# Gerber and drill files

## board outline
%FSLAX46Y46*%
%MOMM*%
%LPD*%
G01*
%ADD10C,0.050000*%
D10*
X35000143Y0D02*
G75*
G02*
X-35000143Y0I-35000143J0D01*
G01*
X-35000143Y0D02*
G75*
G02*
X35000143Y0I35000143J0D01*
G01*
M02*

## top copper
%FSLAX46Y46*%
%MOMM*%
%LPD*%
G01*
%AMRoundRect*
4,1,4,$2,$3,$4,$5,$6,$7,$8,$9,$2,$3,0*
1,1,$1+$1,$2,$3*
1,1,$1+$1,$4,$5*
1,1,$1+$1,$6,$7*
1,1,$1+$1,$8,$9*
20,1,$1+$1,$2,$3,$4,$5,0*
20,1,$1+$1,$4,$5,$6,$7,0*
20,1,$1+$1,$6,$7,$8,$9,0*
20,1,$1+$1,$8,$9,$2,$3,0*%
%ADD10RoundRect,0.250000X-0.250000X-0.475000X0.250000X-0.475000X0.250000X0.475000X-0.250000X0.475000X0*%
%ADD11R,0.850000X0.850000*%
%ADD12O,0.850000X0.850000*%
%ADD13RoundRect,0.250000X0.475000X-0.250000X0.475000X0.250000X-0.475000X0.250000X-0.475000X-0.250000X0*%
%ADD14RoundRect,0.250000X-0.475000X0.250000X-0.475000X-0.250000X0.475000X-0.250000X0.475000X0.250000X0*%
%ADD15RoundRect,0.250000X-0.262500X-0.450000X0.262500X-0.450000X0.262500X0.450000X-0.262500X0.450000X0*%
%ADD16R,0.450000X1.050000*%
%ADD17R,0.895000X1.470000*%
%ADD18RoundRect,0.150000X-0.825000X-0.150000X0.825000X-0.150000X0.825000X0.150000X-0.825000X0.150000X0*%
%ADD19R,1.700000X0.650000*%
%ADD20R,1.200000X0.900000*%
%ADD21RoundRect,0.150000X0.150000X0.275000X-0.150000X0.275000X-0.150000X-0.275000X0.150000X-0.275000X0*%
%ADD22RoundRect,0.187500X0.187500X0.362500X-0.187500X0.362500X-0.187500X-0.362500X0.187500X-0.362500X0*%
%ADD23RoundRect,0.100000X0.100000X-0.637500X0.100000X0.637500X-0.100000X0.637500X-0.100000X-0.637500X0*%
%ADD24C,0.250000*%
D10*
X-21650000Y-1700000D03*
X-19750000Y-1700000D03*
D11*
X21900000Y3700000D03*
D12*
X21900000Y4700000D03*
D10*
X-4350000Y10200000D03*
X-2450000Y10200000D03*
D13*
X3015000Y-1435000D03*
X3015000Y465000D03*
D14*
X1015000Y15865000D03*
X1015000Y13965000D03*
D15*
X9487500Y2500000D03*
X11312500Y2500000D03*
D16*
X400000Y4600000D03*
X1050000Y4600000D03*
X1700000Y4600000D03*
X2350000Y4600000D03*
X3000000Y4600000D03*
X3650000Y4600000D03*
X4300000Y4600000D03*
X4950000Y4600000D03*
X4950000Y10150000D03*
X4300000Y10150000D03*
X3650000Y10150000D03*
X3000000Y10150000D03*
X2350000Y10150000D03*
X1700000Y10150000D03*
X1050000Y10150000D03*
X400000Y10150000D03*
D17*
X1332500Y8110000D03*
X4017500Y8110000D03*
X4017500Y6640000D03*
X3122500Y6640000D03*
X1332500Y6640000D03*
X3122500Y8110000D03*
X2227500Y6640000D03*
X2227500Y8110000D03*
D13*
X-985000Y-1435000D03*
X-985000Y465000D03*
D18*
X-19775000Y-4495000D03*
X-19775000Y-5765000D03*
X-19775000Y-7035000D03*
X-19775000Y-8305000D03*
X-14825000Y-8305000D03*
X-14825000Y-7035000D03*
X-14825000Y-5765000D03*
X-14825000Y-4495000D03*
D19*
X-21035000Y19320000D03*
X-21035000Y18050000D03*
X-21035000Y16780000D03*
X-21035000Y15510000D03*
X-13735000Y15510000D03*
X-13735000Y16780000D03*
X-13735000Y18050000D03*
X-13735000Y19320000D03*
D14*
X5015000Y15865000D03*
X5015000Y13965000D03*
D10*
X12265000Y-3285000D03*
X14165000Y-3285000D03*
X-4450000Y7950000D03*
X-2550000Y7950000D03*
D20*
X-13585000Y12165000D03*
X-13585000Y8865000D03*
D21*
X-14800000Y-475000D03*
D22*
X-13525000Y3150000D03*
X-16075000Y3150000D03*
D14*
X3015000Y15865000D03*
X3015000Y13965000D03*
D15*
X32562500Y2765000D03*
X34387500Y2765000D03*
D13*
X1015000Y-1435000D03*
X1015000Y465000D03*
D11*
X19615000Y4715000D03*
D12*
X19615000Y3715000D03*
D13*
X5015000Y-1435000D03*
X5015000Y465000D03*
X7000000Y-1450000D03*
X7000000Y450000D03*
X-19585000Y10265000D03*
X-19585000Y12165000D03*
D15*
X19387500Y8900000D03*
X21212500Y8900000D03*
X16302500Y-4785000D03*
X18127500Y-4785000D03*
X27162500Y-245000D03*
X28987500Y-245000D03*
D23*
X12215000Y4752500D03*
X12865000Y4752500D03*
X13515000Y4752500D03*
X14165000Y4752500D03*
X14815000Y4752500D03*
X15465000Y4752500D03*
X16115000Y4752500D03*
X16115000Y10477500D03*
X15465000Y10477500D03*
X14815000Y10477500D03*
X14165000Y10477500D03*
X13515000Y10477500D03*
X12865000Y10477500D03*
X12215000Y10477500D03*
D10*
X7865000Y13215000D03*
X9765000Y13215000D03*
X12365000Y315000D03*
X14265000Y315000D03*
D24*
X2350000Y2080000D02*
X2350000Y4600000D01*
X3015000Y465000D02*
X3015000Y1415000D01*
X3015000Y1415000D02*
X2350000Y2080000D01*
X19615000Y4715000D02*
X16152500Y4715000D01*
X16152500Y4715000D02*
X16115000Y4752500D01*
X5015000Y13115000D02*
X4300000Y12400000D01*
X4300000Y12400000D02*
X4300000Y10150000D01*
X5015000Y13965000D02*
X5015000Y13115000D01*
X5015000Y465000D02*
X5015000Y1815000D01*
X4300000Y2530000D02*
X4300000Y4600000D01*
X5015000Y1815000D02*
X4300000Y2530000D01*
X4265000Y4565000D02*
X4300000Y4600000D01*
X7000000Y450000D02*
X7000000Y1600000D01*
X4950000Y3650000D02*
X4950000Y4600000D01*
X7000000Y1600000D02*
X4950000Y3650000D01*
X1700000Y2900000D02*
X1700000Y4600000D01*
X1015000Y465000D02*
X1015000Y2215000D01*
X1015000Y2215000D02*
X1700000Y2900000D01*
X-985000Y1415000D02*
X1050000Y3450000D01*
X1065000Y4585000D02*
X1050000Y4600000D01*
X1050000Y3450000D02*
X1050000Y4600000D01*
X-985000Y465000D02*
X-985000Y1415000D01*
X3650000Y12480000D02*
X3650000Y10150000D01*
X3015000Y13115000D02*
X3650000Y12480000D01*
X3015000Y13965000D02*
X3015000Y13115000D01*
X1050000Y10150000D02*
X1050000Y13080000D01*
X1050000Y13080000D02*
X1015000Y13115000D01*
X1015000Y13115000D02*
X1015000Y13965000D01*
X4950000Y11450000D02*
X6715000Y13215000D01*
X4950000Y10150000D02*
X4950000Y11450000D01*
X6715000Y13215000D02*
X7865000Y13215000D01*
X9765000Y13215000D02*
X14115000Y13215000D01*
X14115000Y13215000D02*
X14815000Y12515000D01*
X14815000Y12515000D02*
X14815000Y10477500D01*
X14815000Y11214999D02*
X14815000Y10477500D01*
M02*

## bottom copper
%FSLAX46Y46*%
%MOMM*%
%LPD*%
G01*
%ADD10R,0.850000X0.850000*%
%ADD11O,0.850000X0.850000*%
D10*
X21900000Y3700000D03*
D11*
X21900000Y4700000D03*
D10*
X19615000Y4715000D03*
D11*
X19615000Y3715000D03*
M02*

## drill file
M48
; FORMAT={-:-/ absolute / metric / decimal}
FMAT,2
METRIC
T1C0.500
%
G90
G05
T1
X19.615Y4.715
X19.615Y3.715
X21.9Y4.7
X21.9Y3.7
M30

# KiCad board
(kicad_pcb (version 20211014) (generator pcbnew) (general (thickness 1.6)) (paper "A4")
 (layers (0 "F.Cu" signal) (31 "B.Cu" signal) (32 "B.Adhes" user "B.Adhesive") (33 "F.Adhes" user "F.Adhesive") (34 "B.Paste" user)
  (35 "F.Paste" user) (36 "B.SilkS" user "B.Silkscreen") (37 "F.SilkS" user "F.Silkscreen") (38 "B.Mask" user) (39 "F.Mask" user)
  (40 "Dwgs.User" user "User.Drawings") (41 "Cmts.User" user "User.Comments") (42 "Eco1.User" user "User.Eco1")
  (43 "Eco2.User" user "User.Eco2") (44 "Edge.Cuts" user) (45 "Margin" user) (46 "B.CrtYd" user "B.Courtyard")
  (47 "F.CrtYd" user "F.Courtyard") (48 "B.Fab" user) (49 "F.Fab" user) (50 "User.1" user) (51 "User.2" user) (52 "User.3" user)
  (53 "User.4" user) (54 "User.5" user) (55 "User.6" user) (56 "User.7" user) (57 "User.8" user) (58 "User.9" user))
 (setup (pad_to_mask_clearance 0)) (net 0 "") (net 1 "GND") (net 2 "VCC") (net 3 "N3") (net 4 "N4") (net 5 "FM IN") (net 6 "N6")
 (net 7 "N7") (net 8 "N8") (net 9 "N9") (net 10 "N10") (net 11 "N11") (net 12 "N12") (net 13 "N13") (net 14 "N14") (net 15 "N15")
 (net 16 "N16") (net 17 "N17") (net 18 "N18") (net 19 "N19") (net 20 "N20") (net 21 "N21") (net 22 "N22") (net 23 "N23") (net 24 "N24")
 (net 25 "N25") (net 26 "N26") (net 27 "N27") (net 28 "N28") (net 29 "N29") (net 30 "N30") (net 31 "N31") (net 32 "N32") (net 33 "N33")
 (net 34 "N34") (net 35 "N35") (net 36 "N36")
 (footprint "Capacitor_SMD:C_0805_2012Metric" (layer "F.Cu") (at -20.7 1.7)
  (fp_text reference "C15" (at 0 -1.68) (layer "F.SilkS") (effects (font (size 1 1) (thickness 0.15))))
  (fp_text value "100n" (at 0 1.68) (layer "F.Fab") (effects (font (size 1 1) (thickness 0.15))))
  (pad "1" smd roundrect locked (at -0.95 0) (size 1 1.45) (layers "F.Cu" "F.Paste" "F.Mask") (roundrect_rratio 0.25) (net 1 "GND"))
  (pad "2" smd roundrect locked (at 0.95 0) (size 1 1.45) (layers "F.Cu" "F.Paste" "F.Mask") (roundrect_rratio 0.25) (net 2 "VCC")))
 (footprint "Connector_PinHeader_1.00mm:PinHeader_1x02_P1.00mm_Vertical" (layer "F.Cu") (at 21.9 -3.7 180)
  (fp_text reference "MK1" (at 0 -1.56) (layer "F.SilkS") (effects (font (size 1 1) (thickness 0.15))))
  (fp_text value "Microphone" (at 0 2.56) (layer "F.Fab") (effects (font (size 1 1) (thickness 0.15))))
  (pad "1" thru_hole rect locked (at 0 0 180) (size 0.85 0.85) (drill 0.5) (layers *.Cu *.Mask) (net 1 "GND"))
  (pad "2" thru_hole oval locked (at 0 1 180) (size 0.85 0.85) (drill 0.5) (layers *.Cu *.Mask) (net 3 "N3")))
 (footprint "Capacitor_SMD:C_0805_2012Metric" (layer "F.Cu") (at -3.4 -10.2)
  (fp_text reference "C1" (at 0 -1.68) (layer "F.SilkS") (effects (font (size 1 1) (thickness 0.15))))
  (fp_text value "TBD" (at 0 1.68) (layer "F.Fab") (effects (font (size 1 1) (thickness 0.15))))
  (pad "1" smd roundrect locked (at -0.95 0) (size 1 1.45) (layers "F.Cu" "F.Paste" "F.Mask") (roundrect_rratio 0.25) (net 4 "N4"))
  (pad "2" smd roundrect locked (at 0.95 0) (size 1 1.45) (layers "F.Cu" "F.Paste" "F.Mask") (roundrect_rratio 0.25) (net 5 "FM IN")))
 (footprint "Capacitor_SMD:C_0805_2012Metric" (layer "F.Cu") (at 3.015 0.485 90)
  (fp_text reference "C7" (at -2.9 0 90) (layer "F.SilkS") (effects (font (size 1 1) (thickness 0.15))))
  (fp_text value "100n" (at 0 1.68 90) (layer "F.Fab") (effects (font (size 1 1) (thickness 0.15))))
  (pad "1" smd roundrect locked (at -0.95 0 90) (size 1 1.45) (layers "F.Cu" "F.Paste" "F.Mask") (roundrect_rratio 0.25) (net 1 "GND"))
  (pad "2" smd roundrect locked (at 0.95 0 90) (size 1 1.45) (layers "F.Cu" "F.Paste" "F.Mask") (roundrect_rratio 0.25) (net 2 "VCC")))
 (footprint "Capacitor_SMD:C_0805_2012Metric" (layer "F.Cu") (at 1.015 -14.915 -90)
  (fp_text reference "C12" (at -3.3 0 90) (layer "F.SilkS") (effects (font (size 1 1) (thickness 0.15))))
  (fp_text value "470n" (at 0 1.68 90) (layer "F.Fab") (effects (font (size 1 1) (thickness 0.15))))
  (pad "1" smd roundrect locked (at -0.95 0 270) (size 1 1.45) (layers "F.Cu" "F.Paste" "F.Mask") (roundrect_rratio 0.25) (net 1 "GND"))
  (pad "2" smd roundrect locked (at 0.95 0 270) (size 1 1.45) (layers "F.Cu" "F.Paste" "F.Mask") (roundrect_rratio 0.25) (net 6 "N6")))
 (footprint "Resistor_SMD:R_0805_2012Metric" (layer "F.Cu") (at 10.4 -2.5)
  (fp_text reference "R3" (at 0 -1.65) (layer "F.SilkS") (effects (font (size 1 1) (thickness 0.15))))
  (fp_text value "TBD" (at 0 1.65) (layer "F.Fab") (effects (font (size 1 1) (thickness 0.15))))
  (pad "1" smd roundrect locked (at -0.9125 0) (size 1.025 1.4) (layers "F.Cu" "F.Paste" "F.Mask") (roundrect_rratio 0.243902) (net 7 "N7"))
  (pad "2" smd roundrect locked (at 0.9125 0) (size 1.025 1.4) (layers "F.Cu" "F.Paste" "F.Mask") (roundrect_rratio 0.243902) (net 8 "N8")))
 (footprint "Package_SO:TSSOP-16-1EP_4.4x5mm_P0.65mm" (layer "F.Cu") (at 2.675 -7.375 90)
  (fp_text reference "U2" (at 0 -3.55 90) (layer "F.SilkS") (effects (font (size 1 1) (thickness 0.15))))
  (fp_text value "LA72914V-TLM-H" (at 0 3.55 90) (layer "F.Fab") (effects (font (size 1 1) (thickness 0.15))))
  (pad "1" smd rect locked (at -2.775 -2.275 90) (size 1.05 0.45) (layers "F.Cu" "F.Paste" "F.Mask") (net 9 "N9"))
  (pad "2" smd rect locked (at -2.775 -1.625 90) (size 1.05 0.45) (layers "F.Cu" "F.Paste" "F.Mask") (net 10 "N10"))
  (pad "3" smd rect locked (at -2.775 -0.975 90) (size 1.05 0.45) (layers "F.Cu" "F.Paste" "F.Mask") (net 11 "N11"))
  (pad "4" smd rect locked (at -2.775 -0.325 90) (size 1.05 0.45) (layers "F.Cu" "F.Paste" "F.Mask") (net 2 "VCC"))
  (pad "5" smd rect locked (at -2.775 0.325 90) (size 1.05 0.45) (layers "F.Cu" "F.Paste" "F.Mask") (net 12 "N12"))
  (pad "6" smd rect locked (at -2.775 0.975 90) (size 1.05 0.45) (layers "F.Cu" "F.Paste" "F.Mask") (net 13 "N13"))
  (pad "7" smd rect locked (at -2.775 1.625 90) (size 1.05 0.45) (layers "F.Cu" "F.Paste" "F.Mask") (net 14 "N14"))
  (pad "8" smd rect locked (at -2.775 2.275 90) (size 1.05 0.45) (layers "F.Cu" "F.Paste" "F.Mask") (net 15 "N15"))
  (pad "9" smd rect locked (at 2.775 2.275 90) (size 1.05 0.45) (layers "F.Cu" "F.Paste" "F.Mask") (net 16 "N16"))
  (pad "10" smd rect locked (at 2.775 1.625 90) (size 1.05 0.45) (layers "F.Cu" "F.Paste" "F.Mask") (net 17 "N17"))
  (pad "11" smd rect locked (at 2.775 0.975 90) (size 1.05 0.45) (layers "F.Cu" "F.Paste" "F.Mask") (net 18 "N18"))
  (pad "12" smd rect locked (at 2.775 0.325 90) (size 1.05 0.45) (layers "F.Cu" "F.Paste" "F.Mask") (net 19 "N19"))
  (pad "13" smd rect locked (at 2.775 -0.325 90) (size 1.05 0.45) (layers "F.Cu" "F.Paste" "F.Mask") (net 1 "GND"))
  (pad "14" smd rect locked (at 2.775 -0.975 90) (size 1.05 0.45) (layers "F.Cu" "F.Paste" "F.Mask") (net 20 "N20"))
  (pad "15" smd rect locked (at 2.775 -1.625 90) (size 1.05 0.45) (layers "F.Cu" "F.Paste" "F.Mask") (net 6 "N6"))
  (pad "16" smd rect locked (at 2.775 -2.275 90) (size 1.05 0.45) (layers "F.Cu" "F.Paste" "F.Mask") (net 7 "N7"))
  (pad "17" smd rect locked (at 0.735 -1.3425 90) (size 1.47 0.895) (layers "F.Cu" "F.Paste" "F.Mask") (solder_paste_margin_ratio -0.2))
  (pad "17" smd rect locked (at 0.735 1.3425 90) (size 1.47 0.895) (layers "F.Cu" "F.Paste" "F.Mask") (solder_paste_margin_ratio -0.2))
  (pad "17" smd rect locked (at -0.735 1.3425 90) (size 1.47 0.895) (layers "F.Cu" "F.Paste" "F.Mask") (solder_paste_margin_ratio -0.2))
  (pad "17" smd rect locked (at -0.735 0.4475 90) (size 1.47 0.895) (layers "F.Cu" "F.Paste" "F.Mask") (solder_paste_margin_ratio -0.2))
  (pad "17" smd rect locked (at -0.735 -1.3425 90) (size 1.47 0.895) (layers "F.Cu" "F.Paste" "F.Mask") (solder_paste_margin_ratio -0.2))
  (pad "17" smd rect locked (at 0.735 0.4475 90) (size 1.47 0.895) (layers "F.Cu" "F.Paste" "F.Mask") (solder_paste_margin_ratio -0.2))
  (pad "17" smd rect locked (at -0.735 -0.4475 90) (size 1.47 0.895) (layers "F.Cu" "F.Paste" "F.Mask") (solder_paste_margin_ratio -0.2))
  (pad "17" smd rect locked (at 0.735 -0.4475 90) (size 1.47 0.895) (layers "F.Cu" "F.Paste" "F.Mask") (solder_paste_margin_ratio -0.2)))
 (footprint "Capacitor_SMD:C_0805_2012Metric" (layer "F.Cu") (at -0.985 0.485 90)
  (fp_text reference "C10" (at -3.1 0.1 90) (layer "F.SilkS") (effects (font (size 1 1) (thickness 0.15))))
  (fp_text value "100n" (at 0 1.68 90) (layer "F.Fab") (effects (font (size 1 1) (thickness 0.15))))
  (pad "1" smd roundrect locked (at -0.95 0 90) (size 1 1.45) (layers "F.Cu" "F.Paste" "F.Mask") (roundrect_rratio 0.25) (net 1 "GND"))
  (pad "2" smd roundrect locked (at 0.95 0 90) (size 1 1.45) (layers "F.Cu" "F.Paste" "F.Mask") (roundrect_rratio 0.25) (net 10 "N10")))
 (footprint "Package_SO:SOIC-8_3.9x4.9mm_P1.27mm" (layer "F.Cu") (at -17.3 6.4)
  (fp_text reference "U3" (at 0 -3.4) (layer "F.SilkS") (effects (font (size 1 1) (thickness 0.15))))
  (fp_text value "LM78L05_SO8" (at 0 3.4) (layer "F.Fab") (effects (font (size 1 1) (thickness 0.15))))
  (pad "1" smd roundrect locked (at -2.475 -1.905) (size 1.95 0.6) (layers "F.Cu" "F.Paste" "F.Mask") (roundrect_rratio 0.25) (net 2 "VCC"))
  (pad "2" smd roundrect locked (at -2.475 -0.635) (size 1.95 0.6) (layers "F.Cu" "F.Paste" "F.Mask") (roundrect_rratio 0.25) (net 1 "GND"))
  (pad "3" smd roundrect locked (at -2.475 0.635) (size 1.95 0.6) (layers "F.Cu" "F.Paste" "F.Mask") (roundrect_rratio 0.25) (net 1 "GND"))
  (pad "4" smd roundrect locked (at -2.475 1.905) (size 1.95 0.6) (layers "F.Cu" "F.Paste" "F.Mask") (roundrect_rratio 0.25) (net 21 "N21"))
  (pad "5" smd roundrect locked (at 2.475 1.905) (size 1.95 0.6) (layers "F.Cu" "F.Paste" "F.Mask") (roundrect_rratio 0.25) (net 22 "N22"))
  (pad "6" smd roundrect locked (at 2.475 0.635) (size 1.95 0.6) (layers "F.Cu" "F.Paste" "F.Mask") (roundrect_rratio 0.25) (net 1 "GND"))
  (pad "7" smd roundrect locked (at 2.475 -0.635) (size 1.95 0.6) (layers "F.Cu" "F.Paste" "F.Mask") (roundrect_rratio 0.25) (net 1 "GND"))
  (pad "8" smd roundrect locked (at 2.475 -1.905) (size 1.95 0.6) (layers "F.Cu" "F.Paste" "F.Mask") (roundrect_rratio 0.25) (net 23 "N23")))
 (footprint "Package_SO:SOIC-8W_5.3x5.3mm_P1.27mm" (layer "F.Cu") (at -17.385 -17.415)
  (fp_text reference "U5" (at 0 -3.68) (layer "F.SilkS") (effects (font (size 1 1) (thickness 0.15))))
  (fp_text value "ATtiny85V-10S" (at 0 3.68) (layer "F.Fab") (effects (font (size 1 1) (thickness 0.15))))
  (pad "1" smd rect locked (at -3.65 -1.905) (size 1.7 0.65) (layers "F.Cu" "F.Paste" "F.Mask") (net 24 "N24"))
  (pad "2" smd rect locked (at -3.65 -0.635) (size 1.7 0.65) (layers "F.Cu" "F.Paste" "F.Mask") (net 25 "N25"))
  (pad "3" smd rect locked (at -3.65 0.635) (size 1.7 0.65) (layers "F.Cu" "F.Paste" "F.Mask") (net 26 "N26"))
  (pad "4" smd rect locked (at -3.65 1.905) (size 1.7 0.65) (layers "F.Cu" "F.Paste" "F.Mask") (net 1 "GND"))
  (pad "5" smd rect locked (at 3.65 1.905) (size 1.7 0.65) (layers "F.Cu" "F.Paste" "F.Mask") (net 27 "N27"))
  (pad "6" smd rect locked (at 3.65 0.635) (size 1.7 0.65) (layers "F.Cu" "F.Paste" "F.Mask") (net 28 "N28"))
  (pad "7" smd rect locked (at 3.65 -0.635) (size 1.7 0.65) (layers "F.Cu" "F.Paste" "F.Mask") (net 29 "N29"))
  (pad "8" smd rect locked (at 3.65 -1.905) (size 1.7 0.65) (layers "F.Cu" "F.Paste" "F.Mask") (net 2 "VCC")))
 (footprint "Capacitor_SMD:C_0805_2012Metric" (layer "F.Cu") (at 5.015 -14.915 -90)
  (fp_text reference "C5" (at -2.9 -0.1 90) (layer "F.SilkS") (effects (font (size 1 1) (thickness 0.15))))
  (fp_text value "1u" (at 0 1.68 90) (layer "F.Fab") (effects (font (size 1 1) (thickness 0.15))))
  (pad "1" smd roundrect locked (at -0.95 0 270) (size 1 1.45) (layers "F.Cu" "F.Paste" "F.Mask") (roundrect_rratio 0.25) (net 1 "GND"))
  (pad "2" smd roundrect locked (at 0.95 0 270) (size 1 1.45) (layers "F.Cu" "F.Paste" "F.Mask") (roundrect_rratio 0.25) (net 17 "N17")))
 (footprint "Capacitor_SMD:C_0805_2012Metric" (layer "F.Cu") (at 13.215 3.285)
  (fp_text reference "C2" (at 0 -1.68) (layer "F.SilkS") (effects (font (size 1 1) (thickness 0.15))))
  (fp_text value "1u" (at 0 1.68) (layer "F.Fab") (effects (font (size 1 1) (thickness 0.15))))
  (pad "1" smd roundrect locked (at -0.95 0) (size 1 1.45) (layers "F.Cu" "F.Paste" "F.Mask") (roundrect_rratio 0.25) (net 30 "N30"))
  (pad "2" smd roundrect locked (at 0.95 0) (size 1 1.45) (layers "F.Cu" "F.Paste" "F.Mask") (roundrect_rratio 0.25) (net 3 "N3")))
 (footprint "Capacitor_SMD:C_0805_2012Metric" (layer "F.Cu") (at -3.5 -7.95)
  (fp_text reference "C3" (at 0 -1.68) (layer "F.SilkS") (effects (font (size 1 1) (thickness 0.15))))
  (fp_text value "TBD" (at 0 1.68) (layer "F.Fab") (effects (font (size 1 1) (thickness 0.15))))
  (pad "1" smd roundrect locked (at -0.95 0) (size 1 1.45) (layers "F.Cu" "F.Paste" "F.Mask") (roundrect_rratio 0.25) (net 12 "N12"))
  (pad "2" smd roundrect locked (at 0.95 0) (size 1 1.45) (layers "F.Cu" "F.Paste" "F.Mask") (roundrect_rratio 0.25) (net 1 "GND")))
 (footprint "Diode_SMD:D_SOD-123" (layer "F.Cu") (at -13.585 -10.515 -90)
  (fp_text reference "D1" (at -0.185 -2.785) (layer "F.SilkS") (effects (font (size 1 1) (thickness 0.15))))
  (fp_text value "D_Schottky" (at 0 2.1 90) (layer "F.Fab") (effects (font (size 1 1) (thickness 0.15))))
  (pad "1" smd rect locked (at -1.65 0 270) (size 0.9 1.2) (layers "F.Cu" "F.Paste" "F.Mask") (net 27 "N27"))
  (pad "2" smd rect locked (at 1.65 0 270) (size 0.9 1.2) (layers "F.Cu" "F.Paste" "F.Mask") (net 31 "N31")))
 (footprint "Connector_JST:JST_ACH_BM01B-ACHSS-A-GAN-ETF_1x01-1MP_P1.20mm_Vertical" (layer "F.Cu") (at -14.8 -1.4 180)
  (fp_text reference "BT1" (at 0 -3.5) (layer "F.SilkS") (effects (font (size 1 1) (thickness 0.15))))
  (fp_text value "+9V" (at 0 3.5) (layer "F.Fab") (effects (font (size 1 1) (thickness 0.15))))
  (pad "1" smd roundrect locked (at 0 -1.875 180) (size 0.6 0.85) (layers "F.Cu" "F.Paste" "F.Mask") (roundrect_rratio 0.25) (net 23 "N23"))
  (pad "MP" smd roundrect locked (at -1.275 1.75 180) (size 0.75 1.1) (layers "F.Cu" "F.Paste" "F.Mask") (roundrect_rratio 0.25))
  (pad "MP" smd roundrect locked (at 1.275 1.75 180) (size 0.75 1.1) (layers "F.Cu" "F.Paste" "F.Mask") (roundrect_rratio 0.25)))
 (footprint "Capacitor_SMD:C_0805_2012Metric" (layer "F.Cu") (at 3.015 -14.915 -90)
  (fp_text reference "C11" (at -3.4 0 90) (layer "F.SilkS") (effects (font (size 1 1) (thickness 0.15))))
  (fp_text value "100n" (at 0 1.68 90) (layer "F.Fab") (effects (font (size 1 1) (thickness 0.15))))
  (pad "1" smd roundrect locked (at -0.95 0 270) (size 1 1.45) (layers "F.Cu" "F.Paste" "F.Mask") (roundrect_rratio 0.25) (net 1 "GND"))
  (pad "2" smd roundrect locked (at 0.95 0 270) (size 1 1.45) (layers "F.Cu" "F.Paste" "F.Mask") (roundrect_rratio 0.25) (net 18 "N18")))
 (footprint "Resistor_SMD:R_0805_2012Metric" (layer "F.Cu") (at 33.475 -2.765)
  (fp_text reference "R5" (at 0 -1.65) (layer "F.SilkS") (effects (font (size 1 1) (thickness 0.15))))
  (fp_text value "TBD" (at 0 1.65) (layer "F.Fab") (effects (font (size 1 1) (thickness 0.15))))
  (pad "1" smd roundrect locked (at -0.9125 0) (size 1.025 1.4) (layers "F.Cu" "F.Paste" "F.Mask") (roundrect_rratio 0.243902)
   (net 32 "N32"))
  (pad "2" smd roundrect locked (at 0.9125 0) (size 1.025 1.4) (layers "F.Cu" "F.Paste" "F.Mask") (roundrect_rratio 0.243902) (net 1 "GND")))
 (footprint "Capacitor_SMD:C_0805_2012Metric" (layer "F.Cu") (at 1.015 0.485 90)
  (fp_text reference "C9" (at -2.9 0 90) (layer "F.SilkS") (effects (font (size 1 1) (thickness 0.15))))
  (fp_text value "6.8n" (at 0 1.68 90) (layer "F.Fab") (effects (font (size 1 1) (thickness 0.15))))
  (pad "1" smd roundrect locked (at -0.95 0 90) (size 1 1.45) (layers "F.Cu" "F.Paste" "F.Mask") (roundrect_rratio 0.25) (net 1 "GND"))
  (pad "2" smd roundrect locked (at 0.95 0 90) (size 1 1.45) (layers "F.Cu" "F.Paste" "F.Mask") (roundrect_rratio 0.25) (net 11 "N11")))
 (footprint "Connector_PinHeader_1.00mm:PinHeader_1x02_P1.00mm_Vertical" (layer "F.Cu") (at 19.615 -4.715)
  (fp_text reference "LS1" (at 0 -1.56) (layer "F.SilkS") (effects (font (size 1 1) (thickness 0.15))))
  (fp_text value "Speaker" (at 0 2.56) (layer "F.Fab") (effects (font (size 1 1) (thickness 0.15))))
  (pad "1" thru_hole rect locked (at 0 0) (size 0.85 0.85) (drill 0.5) (layers *.Cu *.Mask) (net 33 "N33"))
  (pad "2" thru_hole oval locked (at 0 1) (size 0.85 0.85) (drill 0.5) (layers *.Cu *.Mask) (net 1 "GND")))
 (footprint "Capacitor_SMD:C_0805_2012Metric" (layer "F.Cu") (at 5.015 0.485 90)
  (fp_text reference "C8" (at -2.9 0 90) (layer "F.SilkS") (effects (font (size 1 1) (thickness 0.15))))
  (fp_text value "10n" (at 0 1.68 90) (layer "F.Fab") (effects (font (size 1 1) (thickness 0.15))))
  (pad "1" smd roundrect locked (at -0.95 0 90) (size 1 1.45) (layers "F.Cu" "F.Paste" "F.Mask") (roundrect_rratio 0.25) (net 1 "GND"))
  (pad "2" smd roundrect locked (at 0.95 0 90) (size 1 1.45) (layers "F.Cu" "F.Paste" "F.Mask") (roundrect_rratio 0.25) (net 14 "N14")))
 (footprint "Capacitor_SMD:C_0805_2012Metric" (layer "F.Cu") (at 7 0.5 90)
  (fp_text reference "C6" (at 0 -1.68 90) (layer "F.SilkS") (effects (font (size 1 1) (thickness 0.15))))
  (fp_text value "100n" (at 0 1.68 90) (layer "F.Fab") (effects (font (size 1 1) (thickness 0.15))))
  (pad "1" smd roundrect locked (at -0.95 0 90) (size 1 1.45) (layers "F.Cu" "F.Paste" "F.Mask") (roundrect_rratio 0.25) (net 14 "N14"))
  (pad "2" smd roundrect locked (at 0.95 0 90) (size 1 1.45) (layers "F.Cu" "F.Paste" "F.Mask") (roundrect_rratio 0.25) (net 15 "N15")))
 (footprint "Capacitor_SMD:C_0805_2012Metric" (layer "F.Cu") (at -19.585 -11.215 90)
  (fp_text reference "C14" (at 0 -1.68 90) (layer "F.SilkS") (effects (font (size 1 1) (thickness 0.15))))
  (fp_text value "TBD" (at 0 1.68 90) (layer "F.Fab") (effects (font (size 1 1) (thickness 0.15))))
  (pad "1" smd roundrect locked (at -0.95 0 90) (size 1 1.45) (layers "F.Cu" "F.Paste" "F.Mask") (roundrect_rratio 0.25) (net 1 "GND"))
  (pad "2" smd roundrect locked (at 0.95 0 90) (size 1 1.45) (layers "F.Cu" "F.Paste" "F.Mask") (roundrect_rratio 0.25) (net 27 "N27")))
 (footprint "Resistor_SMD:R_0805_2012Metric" (layer "F.Cu") (at 20.3 -8.9)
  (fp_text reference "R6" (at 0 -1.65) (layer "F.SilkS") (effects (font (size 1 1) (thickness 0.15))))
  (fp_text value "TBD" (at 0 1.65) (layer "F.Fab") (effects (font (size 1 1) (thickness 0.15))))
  (pad "1" smd roundrect locked (at -0.9125 0) (size 1.025 1.4) (layers "F.Cu" "F.Paste" "F.Mask") (roundrect_rratio 0.243902)
   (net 33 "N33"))
  (pad "2" smd roundrect locked (at 0.9125 0) (size 1.025 1.4) (layers "F.Cu" "F.Paste" "F.Mask") (roundrect_rratio 0.243902) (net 32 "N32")))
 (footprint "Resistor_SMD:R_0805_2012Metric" (layer "F.Cu") (at 17.215 4.785)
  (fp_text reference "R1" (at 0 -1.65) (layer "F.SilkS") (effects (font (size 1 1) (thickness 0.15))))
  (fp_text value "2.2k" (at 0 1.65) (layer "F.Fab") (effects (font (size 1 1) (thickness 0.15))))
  (pad "1" smd roundrect locked (at -0.9125 0) (size 1.025 1.4) (layers "F.Cu" "F.Paste" "F.Mask") (roundrect_rratio 0.243902) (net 3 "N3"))
  (pad "2" smd roundrect locked (at 0.9125 0) (size 1.025 1.4) (layers "F.Cu" "F.Paste" "F.Mask") (roundrect_rratio 0.243902) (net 2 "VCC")))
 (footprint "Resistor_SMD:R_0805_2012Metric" (layer "F.Cu") (at 28.075 0.245)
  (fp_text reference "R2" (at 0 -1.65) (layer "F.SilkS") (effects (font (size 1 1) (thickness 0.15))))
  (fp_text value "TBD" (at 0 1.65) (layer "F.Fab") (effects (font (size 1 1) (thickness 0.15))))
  (pad "1" smd roundrect locked (at -0.9125 0) (size 1.025 1.4) (layers "F.Cu" "F.Paste" "F.Mask") (roundrect_rratio 0.243902) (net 1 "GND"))
  (pad "2" smd roundrect locked (at 0.9125 0) (size 1.025 1.4) (layers "F.Cu" "F.Paste" "F.Mask") (roundrect_rratio 0.243902) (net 8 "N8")))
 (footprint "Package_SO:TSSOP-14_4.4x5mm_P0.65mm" (layer "F.Cu") (at 14.165 -7.615 90)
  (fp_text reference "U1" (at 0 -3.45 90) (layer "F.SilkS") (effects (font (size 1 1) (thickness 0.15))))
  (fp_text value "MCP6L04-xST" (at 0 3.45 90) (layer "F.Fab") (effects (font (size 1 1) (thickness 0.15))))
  (pad "1" smd roundrect locked (at -2.8625 -1.95 90) (size 1.475 0.4) (layers "F.Cu" "F.Paste" "F.Mask") (roundrect_rratio 0.25)
   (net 7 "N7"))
  (pad "2" smd roundrect locked (at -2.8625 -1.3 90) (size 1.475 0.4) (layers "F.Cu" "F.Paste" "F.Mask") (roundrect_rratio 0.25)
   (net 8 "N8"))
  (pad "3" smd roundrect locked (at -2.8625 -0.65 90) (size 1.475 0.4) (layers "F.Cu" "F.Paste" "F.Mask") (roundrect_rratio 0.25)
   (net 30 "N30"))
  (pad "4" smd roundrect locked (at -2.8625 0 90) (size 1.475 0.4) (layers "F.Cu" "F.Paste" "F.Mask") (roundrect_rratio 0.25) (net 2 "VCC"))
  (pad "5" smd roundrect locked (at -2.8625 0.65 90) (size 1.475 0.4) (layers "F.Cu" "F.Paste" "F.Mask") (roundrect_rratio 0.25)
   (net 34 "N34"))
  (pad "6" smd roundrect locked (at -2.8625 1.3 90) (size 1.475 0.4) (layers "F.Cu" "F.Paste" "F.Mask") (roundrect_rratio 0.25)
   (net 32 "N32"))
  (pad "7" smd roundrect locked (at -2.8625 1.95 90) (size 1.475 0.4) (layers "F.Cu" "F.Paste" "F.Mask") (roundrect_rratio 0.25)
   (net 33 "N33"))
  (pad "8" smd roundrect locked (at 2.8625 1.95 90) (size 1.475 0.4) (layers "F.Cu" "F.Paste" "F.Mask") (roundrect_rratio 0.25)
   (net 31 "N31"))
  (pad "9" smd roundrect locked (at 2.8625 1.3 90) (size 1.475 0.4) (layers "F.Cu" "F.Paste" "F.Mask") (roundrect_rratio 0.25)
   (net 31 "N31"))
  (pad "10" smd roundrect locked (at 2.8625 0.65 90) (size 1.475 0.4) (layers "F.Cu" "F.Paste" "F.Mask") (roundrect_rratio 0.25)
   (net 34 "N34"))
  (pad "11" smd roundrect locked (at 2.8625 0 90) (size 1.475 0.4) (layers "F.Cu" "F.Paste" "F.Mask") (roundrect_rratio 0.25) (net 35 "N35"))
  (pad "12" smd roundrect locked (at 2.8625 -0.65 90) (size 1.475 0.4) (layers "F.Cu" "F.Paste" "F.Mask") (roundrect_rratio 0.25))
  (pad "13" smd roundrect locked (at 2.8625 -1.3 90) (size 1.475 0.4) (layers "F.Cu" "F.Paste" "F.Mask") (roundrect_rratio 0.25))
  (pad "14" smd roundrect locked (at 2.8625 -1.95 90) (size 1.475 0.4) (layers "F.Cu" "F.Paste" "F.Mask") (roundrect_rratio 0.25)))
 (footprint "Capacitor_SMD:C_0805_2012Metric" (layer "F.Cu") (at 8.815 -13.215)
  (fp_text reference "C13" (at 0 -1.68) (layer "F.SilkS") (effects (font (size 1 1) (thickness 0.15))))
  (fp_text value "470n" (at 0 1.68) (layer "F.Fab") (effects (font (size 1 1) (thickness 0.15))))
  (pad "1" smd roundrect locked (at -0.95 0) (size 1 1.45) (layers "F.Cu" "F.Paste" "F.Mask") (roundrect_rratio 0.25) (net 16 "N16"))
  (pad "2" smd roundrect locked (at 0.95 0) (size 1 1.45) (layers "F.Cu" "F.Paste" "F.Mask") (roundrect_rratio 0.25) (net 34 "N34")))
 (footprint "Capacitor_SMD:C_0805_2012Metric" (layer "F.Cu") (at 13.315 -0.315)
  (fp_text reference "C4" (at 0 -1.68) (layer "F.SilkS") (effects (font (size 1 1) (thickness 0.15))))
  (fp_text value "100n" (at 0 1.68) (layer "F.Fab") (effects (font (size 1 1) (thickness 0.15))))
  (pad "1" smd roundrect locked (at -0.95 0) (size 1 1.45) (layers "F.Cu" "F.Paste" "F.Mask") (roundrect_rratio 0.25) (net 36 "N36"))
  (pad "2" smd roundrect locked (at 0.95 0) (size 1 1.45) (layers "F.Cu" "F.Paste" "F.Mask") (roundrect_rratio 0.25) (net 2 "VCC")))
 (gr_circle (center 0 0) (end -35 -0.1) (layer "Edge.Cuts") (width 0.05) (fill none))
 (segment (start 2.35 -2.08) (end 2.35 -4.6) (width 0.25) (layer "F.Cu") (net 2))
 (segment (start 3.015 -0.465) (end 3.015 -1.415) (width 0.25) (layer "F.Cu") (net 2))
 (segment (start 3.015 -1.415) (end 2.35 -2.08) (width 0.25) (layer "F.Cu") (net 2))
 (segment (start 19.615 -4.715) (end 16.1525 -4.715) (width 0.25) (layer "F.Cu") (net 33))
 (segment (start 16.1525 -4.715) (end 16.115 -4.7525) (width 0.25) (layer "F.Cu") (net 33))
 (segment (start 5.015 -13.115) (end 4.3 -12.4) (width 0.25) (layer "F.Cu") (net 17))
 (segment (start 4.3 -12.4) (end 4.3 -10.15) (width 0.25) (layer "F.Cu") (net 17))
 (segment (start 5.015 -13.965) (end 5.015 -13.115) (width 0.25) (layer "F.Cu") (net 17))
 (segment (start 5.015 -0.465) (end 5.015 -1.815) (width 0.25) (layer "F.Cu") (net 14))
 (segment (start 4.3 -2.53) (end 4.3 -4.6) (width 0.25) (layer "F.Cu") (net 14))
 (segment (start 5.015 -1.815) (end 4.3 -2.53) (width 0.25) (layer "F.Cu") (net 14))
 (segment (start 4.265 -4.565) (end 4.3 -4.6) (width 0.25) (layer "F.Cu") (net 14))
 (segment (start 7 -0.45) (end 7 -1.6) (width 0.25) (layer "F.Cu") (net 15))
 (segment (start 4.95 -3.65) (end 4.95 -4.6) (width 0.25) (layer "F.Cu") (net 15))
 (segment (start 7 -1.6) (end 4.95 -3.65) (width 0.25) (layer "F.Cu") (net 15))
 (segment (start 1.7 -2.9) (end 1.7 -4.6) (width 0.25) (layer "F.Cu") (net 11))
 (segment (start 1.015 -0.465) (end 1.015 -2.215) (width 0.25) (layer "F.Cu") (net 11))
 (segment (start 1.015 -2.215) (end 1.7 -2.9) (width 0.25) (layer "F.Cu") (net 11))
 (segment (start -0.985 -1.415) (end 1.05 -3.45) (width 0.25) (layer "F.Cu") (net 10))
 (segment (start 1.065 -4.585) (end 1.05 -4.6) (width 0.25) (layer "F.Cu") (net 10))
 (segment (start 1.05 -3.45) (end 1.05 -4.6) (width 0.25) (layer "F.Cu") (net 10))
 (segment (start -0.985 -0.465) (end -0.985 -1.415) (width 0.25) (layer "F.Cu") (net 10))
 (segment (start 3.65 -12.48) (end 3.65 -10.15) (width 0.25) (layer "F.Cu") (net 18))
 (segment (start 3.015 -13.115) (end 3.65 -12.48) (width 0.25) (layer "F.Cu") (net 18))
 (segment (start 3.015 -13.965) (end 3.015 -13.115) (width 0.25) (layer "F.Cu") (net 18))
 (segment (start 1.05 -10.15) (end 1.05 -13.08) (width 0.25) (layer "F.Cu") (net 6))
 (segment (start 1.05 -13.08) (end 1.015 -13.115) (width 0.25) (layer "F.Cu") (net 6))
 (segment (start 1.015 -13.115) (end 1.015 -13.965) (width 0.25) (layer "F.Cu") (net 6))
 (segment (start 4.95 -11.45) (end 6.715 -13.215) (width 0.25) (layer "F.Cu") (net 16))
 (segment (start 4.95 -10.15) (end 4.95 -11.45) (width 0.25) (layer "F.Cu") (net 16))
 (segment (start 6.715 -13.215) (end 7.865 -13.215) (width 0.25) (layer "F.Cu") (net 16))
 (segment (start 9.765 -13.215) (end 14.115 -13.215) (width 0.25) (layer "F.Cu") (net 34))
 (segment (start 14.115 -13.215) (end 14.815 -12.515) (width 0.25) (layer "F.Cu") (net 34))
 (segment (start 14.815 -12.515) (end 14.815 -10.4775) (width 0.25) (layer "F.Cu") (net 34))
 (segment (start 14.815 -11.214999) (end 14.815 -10.4775) (width 0.25) (layer "F.Cu") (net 34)))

